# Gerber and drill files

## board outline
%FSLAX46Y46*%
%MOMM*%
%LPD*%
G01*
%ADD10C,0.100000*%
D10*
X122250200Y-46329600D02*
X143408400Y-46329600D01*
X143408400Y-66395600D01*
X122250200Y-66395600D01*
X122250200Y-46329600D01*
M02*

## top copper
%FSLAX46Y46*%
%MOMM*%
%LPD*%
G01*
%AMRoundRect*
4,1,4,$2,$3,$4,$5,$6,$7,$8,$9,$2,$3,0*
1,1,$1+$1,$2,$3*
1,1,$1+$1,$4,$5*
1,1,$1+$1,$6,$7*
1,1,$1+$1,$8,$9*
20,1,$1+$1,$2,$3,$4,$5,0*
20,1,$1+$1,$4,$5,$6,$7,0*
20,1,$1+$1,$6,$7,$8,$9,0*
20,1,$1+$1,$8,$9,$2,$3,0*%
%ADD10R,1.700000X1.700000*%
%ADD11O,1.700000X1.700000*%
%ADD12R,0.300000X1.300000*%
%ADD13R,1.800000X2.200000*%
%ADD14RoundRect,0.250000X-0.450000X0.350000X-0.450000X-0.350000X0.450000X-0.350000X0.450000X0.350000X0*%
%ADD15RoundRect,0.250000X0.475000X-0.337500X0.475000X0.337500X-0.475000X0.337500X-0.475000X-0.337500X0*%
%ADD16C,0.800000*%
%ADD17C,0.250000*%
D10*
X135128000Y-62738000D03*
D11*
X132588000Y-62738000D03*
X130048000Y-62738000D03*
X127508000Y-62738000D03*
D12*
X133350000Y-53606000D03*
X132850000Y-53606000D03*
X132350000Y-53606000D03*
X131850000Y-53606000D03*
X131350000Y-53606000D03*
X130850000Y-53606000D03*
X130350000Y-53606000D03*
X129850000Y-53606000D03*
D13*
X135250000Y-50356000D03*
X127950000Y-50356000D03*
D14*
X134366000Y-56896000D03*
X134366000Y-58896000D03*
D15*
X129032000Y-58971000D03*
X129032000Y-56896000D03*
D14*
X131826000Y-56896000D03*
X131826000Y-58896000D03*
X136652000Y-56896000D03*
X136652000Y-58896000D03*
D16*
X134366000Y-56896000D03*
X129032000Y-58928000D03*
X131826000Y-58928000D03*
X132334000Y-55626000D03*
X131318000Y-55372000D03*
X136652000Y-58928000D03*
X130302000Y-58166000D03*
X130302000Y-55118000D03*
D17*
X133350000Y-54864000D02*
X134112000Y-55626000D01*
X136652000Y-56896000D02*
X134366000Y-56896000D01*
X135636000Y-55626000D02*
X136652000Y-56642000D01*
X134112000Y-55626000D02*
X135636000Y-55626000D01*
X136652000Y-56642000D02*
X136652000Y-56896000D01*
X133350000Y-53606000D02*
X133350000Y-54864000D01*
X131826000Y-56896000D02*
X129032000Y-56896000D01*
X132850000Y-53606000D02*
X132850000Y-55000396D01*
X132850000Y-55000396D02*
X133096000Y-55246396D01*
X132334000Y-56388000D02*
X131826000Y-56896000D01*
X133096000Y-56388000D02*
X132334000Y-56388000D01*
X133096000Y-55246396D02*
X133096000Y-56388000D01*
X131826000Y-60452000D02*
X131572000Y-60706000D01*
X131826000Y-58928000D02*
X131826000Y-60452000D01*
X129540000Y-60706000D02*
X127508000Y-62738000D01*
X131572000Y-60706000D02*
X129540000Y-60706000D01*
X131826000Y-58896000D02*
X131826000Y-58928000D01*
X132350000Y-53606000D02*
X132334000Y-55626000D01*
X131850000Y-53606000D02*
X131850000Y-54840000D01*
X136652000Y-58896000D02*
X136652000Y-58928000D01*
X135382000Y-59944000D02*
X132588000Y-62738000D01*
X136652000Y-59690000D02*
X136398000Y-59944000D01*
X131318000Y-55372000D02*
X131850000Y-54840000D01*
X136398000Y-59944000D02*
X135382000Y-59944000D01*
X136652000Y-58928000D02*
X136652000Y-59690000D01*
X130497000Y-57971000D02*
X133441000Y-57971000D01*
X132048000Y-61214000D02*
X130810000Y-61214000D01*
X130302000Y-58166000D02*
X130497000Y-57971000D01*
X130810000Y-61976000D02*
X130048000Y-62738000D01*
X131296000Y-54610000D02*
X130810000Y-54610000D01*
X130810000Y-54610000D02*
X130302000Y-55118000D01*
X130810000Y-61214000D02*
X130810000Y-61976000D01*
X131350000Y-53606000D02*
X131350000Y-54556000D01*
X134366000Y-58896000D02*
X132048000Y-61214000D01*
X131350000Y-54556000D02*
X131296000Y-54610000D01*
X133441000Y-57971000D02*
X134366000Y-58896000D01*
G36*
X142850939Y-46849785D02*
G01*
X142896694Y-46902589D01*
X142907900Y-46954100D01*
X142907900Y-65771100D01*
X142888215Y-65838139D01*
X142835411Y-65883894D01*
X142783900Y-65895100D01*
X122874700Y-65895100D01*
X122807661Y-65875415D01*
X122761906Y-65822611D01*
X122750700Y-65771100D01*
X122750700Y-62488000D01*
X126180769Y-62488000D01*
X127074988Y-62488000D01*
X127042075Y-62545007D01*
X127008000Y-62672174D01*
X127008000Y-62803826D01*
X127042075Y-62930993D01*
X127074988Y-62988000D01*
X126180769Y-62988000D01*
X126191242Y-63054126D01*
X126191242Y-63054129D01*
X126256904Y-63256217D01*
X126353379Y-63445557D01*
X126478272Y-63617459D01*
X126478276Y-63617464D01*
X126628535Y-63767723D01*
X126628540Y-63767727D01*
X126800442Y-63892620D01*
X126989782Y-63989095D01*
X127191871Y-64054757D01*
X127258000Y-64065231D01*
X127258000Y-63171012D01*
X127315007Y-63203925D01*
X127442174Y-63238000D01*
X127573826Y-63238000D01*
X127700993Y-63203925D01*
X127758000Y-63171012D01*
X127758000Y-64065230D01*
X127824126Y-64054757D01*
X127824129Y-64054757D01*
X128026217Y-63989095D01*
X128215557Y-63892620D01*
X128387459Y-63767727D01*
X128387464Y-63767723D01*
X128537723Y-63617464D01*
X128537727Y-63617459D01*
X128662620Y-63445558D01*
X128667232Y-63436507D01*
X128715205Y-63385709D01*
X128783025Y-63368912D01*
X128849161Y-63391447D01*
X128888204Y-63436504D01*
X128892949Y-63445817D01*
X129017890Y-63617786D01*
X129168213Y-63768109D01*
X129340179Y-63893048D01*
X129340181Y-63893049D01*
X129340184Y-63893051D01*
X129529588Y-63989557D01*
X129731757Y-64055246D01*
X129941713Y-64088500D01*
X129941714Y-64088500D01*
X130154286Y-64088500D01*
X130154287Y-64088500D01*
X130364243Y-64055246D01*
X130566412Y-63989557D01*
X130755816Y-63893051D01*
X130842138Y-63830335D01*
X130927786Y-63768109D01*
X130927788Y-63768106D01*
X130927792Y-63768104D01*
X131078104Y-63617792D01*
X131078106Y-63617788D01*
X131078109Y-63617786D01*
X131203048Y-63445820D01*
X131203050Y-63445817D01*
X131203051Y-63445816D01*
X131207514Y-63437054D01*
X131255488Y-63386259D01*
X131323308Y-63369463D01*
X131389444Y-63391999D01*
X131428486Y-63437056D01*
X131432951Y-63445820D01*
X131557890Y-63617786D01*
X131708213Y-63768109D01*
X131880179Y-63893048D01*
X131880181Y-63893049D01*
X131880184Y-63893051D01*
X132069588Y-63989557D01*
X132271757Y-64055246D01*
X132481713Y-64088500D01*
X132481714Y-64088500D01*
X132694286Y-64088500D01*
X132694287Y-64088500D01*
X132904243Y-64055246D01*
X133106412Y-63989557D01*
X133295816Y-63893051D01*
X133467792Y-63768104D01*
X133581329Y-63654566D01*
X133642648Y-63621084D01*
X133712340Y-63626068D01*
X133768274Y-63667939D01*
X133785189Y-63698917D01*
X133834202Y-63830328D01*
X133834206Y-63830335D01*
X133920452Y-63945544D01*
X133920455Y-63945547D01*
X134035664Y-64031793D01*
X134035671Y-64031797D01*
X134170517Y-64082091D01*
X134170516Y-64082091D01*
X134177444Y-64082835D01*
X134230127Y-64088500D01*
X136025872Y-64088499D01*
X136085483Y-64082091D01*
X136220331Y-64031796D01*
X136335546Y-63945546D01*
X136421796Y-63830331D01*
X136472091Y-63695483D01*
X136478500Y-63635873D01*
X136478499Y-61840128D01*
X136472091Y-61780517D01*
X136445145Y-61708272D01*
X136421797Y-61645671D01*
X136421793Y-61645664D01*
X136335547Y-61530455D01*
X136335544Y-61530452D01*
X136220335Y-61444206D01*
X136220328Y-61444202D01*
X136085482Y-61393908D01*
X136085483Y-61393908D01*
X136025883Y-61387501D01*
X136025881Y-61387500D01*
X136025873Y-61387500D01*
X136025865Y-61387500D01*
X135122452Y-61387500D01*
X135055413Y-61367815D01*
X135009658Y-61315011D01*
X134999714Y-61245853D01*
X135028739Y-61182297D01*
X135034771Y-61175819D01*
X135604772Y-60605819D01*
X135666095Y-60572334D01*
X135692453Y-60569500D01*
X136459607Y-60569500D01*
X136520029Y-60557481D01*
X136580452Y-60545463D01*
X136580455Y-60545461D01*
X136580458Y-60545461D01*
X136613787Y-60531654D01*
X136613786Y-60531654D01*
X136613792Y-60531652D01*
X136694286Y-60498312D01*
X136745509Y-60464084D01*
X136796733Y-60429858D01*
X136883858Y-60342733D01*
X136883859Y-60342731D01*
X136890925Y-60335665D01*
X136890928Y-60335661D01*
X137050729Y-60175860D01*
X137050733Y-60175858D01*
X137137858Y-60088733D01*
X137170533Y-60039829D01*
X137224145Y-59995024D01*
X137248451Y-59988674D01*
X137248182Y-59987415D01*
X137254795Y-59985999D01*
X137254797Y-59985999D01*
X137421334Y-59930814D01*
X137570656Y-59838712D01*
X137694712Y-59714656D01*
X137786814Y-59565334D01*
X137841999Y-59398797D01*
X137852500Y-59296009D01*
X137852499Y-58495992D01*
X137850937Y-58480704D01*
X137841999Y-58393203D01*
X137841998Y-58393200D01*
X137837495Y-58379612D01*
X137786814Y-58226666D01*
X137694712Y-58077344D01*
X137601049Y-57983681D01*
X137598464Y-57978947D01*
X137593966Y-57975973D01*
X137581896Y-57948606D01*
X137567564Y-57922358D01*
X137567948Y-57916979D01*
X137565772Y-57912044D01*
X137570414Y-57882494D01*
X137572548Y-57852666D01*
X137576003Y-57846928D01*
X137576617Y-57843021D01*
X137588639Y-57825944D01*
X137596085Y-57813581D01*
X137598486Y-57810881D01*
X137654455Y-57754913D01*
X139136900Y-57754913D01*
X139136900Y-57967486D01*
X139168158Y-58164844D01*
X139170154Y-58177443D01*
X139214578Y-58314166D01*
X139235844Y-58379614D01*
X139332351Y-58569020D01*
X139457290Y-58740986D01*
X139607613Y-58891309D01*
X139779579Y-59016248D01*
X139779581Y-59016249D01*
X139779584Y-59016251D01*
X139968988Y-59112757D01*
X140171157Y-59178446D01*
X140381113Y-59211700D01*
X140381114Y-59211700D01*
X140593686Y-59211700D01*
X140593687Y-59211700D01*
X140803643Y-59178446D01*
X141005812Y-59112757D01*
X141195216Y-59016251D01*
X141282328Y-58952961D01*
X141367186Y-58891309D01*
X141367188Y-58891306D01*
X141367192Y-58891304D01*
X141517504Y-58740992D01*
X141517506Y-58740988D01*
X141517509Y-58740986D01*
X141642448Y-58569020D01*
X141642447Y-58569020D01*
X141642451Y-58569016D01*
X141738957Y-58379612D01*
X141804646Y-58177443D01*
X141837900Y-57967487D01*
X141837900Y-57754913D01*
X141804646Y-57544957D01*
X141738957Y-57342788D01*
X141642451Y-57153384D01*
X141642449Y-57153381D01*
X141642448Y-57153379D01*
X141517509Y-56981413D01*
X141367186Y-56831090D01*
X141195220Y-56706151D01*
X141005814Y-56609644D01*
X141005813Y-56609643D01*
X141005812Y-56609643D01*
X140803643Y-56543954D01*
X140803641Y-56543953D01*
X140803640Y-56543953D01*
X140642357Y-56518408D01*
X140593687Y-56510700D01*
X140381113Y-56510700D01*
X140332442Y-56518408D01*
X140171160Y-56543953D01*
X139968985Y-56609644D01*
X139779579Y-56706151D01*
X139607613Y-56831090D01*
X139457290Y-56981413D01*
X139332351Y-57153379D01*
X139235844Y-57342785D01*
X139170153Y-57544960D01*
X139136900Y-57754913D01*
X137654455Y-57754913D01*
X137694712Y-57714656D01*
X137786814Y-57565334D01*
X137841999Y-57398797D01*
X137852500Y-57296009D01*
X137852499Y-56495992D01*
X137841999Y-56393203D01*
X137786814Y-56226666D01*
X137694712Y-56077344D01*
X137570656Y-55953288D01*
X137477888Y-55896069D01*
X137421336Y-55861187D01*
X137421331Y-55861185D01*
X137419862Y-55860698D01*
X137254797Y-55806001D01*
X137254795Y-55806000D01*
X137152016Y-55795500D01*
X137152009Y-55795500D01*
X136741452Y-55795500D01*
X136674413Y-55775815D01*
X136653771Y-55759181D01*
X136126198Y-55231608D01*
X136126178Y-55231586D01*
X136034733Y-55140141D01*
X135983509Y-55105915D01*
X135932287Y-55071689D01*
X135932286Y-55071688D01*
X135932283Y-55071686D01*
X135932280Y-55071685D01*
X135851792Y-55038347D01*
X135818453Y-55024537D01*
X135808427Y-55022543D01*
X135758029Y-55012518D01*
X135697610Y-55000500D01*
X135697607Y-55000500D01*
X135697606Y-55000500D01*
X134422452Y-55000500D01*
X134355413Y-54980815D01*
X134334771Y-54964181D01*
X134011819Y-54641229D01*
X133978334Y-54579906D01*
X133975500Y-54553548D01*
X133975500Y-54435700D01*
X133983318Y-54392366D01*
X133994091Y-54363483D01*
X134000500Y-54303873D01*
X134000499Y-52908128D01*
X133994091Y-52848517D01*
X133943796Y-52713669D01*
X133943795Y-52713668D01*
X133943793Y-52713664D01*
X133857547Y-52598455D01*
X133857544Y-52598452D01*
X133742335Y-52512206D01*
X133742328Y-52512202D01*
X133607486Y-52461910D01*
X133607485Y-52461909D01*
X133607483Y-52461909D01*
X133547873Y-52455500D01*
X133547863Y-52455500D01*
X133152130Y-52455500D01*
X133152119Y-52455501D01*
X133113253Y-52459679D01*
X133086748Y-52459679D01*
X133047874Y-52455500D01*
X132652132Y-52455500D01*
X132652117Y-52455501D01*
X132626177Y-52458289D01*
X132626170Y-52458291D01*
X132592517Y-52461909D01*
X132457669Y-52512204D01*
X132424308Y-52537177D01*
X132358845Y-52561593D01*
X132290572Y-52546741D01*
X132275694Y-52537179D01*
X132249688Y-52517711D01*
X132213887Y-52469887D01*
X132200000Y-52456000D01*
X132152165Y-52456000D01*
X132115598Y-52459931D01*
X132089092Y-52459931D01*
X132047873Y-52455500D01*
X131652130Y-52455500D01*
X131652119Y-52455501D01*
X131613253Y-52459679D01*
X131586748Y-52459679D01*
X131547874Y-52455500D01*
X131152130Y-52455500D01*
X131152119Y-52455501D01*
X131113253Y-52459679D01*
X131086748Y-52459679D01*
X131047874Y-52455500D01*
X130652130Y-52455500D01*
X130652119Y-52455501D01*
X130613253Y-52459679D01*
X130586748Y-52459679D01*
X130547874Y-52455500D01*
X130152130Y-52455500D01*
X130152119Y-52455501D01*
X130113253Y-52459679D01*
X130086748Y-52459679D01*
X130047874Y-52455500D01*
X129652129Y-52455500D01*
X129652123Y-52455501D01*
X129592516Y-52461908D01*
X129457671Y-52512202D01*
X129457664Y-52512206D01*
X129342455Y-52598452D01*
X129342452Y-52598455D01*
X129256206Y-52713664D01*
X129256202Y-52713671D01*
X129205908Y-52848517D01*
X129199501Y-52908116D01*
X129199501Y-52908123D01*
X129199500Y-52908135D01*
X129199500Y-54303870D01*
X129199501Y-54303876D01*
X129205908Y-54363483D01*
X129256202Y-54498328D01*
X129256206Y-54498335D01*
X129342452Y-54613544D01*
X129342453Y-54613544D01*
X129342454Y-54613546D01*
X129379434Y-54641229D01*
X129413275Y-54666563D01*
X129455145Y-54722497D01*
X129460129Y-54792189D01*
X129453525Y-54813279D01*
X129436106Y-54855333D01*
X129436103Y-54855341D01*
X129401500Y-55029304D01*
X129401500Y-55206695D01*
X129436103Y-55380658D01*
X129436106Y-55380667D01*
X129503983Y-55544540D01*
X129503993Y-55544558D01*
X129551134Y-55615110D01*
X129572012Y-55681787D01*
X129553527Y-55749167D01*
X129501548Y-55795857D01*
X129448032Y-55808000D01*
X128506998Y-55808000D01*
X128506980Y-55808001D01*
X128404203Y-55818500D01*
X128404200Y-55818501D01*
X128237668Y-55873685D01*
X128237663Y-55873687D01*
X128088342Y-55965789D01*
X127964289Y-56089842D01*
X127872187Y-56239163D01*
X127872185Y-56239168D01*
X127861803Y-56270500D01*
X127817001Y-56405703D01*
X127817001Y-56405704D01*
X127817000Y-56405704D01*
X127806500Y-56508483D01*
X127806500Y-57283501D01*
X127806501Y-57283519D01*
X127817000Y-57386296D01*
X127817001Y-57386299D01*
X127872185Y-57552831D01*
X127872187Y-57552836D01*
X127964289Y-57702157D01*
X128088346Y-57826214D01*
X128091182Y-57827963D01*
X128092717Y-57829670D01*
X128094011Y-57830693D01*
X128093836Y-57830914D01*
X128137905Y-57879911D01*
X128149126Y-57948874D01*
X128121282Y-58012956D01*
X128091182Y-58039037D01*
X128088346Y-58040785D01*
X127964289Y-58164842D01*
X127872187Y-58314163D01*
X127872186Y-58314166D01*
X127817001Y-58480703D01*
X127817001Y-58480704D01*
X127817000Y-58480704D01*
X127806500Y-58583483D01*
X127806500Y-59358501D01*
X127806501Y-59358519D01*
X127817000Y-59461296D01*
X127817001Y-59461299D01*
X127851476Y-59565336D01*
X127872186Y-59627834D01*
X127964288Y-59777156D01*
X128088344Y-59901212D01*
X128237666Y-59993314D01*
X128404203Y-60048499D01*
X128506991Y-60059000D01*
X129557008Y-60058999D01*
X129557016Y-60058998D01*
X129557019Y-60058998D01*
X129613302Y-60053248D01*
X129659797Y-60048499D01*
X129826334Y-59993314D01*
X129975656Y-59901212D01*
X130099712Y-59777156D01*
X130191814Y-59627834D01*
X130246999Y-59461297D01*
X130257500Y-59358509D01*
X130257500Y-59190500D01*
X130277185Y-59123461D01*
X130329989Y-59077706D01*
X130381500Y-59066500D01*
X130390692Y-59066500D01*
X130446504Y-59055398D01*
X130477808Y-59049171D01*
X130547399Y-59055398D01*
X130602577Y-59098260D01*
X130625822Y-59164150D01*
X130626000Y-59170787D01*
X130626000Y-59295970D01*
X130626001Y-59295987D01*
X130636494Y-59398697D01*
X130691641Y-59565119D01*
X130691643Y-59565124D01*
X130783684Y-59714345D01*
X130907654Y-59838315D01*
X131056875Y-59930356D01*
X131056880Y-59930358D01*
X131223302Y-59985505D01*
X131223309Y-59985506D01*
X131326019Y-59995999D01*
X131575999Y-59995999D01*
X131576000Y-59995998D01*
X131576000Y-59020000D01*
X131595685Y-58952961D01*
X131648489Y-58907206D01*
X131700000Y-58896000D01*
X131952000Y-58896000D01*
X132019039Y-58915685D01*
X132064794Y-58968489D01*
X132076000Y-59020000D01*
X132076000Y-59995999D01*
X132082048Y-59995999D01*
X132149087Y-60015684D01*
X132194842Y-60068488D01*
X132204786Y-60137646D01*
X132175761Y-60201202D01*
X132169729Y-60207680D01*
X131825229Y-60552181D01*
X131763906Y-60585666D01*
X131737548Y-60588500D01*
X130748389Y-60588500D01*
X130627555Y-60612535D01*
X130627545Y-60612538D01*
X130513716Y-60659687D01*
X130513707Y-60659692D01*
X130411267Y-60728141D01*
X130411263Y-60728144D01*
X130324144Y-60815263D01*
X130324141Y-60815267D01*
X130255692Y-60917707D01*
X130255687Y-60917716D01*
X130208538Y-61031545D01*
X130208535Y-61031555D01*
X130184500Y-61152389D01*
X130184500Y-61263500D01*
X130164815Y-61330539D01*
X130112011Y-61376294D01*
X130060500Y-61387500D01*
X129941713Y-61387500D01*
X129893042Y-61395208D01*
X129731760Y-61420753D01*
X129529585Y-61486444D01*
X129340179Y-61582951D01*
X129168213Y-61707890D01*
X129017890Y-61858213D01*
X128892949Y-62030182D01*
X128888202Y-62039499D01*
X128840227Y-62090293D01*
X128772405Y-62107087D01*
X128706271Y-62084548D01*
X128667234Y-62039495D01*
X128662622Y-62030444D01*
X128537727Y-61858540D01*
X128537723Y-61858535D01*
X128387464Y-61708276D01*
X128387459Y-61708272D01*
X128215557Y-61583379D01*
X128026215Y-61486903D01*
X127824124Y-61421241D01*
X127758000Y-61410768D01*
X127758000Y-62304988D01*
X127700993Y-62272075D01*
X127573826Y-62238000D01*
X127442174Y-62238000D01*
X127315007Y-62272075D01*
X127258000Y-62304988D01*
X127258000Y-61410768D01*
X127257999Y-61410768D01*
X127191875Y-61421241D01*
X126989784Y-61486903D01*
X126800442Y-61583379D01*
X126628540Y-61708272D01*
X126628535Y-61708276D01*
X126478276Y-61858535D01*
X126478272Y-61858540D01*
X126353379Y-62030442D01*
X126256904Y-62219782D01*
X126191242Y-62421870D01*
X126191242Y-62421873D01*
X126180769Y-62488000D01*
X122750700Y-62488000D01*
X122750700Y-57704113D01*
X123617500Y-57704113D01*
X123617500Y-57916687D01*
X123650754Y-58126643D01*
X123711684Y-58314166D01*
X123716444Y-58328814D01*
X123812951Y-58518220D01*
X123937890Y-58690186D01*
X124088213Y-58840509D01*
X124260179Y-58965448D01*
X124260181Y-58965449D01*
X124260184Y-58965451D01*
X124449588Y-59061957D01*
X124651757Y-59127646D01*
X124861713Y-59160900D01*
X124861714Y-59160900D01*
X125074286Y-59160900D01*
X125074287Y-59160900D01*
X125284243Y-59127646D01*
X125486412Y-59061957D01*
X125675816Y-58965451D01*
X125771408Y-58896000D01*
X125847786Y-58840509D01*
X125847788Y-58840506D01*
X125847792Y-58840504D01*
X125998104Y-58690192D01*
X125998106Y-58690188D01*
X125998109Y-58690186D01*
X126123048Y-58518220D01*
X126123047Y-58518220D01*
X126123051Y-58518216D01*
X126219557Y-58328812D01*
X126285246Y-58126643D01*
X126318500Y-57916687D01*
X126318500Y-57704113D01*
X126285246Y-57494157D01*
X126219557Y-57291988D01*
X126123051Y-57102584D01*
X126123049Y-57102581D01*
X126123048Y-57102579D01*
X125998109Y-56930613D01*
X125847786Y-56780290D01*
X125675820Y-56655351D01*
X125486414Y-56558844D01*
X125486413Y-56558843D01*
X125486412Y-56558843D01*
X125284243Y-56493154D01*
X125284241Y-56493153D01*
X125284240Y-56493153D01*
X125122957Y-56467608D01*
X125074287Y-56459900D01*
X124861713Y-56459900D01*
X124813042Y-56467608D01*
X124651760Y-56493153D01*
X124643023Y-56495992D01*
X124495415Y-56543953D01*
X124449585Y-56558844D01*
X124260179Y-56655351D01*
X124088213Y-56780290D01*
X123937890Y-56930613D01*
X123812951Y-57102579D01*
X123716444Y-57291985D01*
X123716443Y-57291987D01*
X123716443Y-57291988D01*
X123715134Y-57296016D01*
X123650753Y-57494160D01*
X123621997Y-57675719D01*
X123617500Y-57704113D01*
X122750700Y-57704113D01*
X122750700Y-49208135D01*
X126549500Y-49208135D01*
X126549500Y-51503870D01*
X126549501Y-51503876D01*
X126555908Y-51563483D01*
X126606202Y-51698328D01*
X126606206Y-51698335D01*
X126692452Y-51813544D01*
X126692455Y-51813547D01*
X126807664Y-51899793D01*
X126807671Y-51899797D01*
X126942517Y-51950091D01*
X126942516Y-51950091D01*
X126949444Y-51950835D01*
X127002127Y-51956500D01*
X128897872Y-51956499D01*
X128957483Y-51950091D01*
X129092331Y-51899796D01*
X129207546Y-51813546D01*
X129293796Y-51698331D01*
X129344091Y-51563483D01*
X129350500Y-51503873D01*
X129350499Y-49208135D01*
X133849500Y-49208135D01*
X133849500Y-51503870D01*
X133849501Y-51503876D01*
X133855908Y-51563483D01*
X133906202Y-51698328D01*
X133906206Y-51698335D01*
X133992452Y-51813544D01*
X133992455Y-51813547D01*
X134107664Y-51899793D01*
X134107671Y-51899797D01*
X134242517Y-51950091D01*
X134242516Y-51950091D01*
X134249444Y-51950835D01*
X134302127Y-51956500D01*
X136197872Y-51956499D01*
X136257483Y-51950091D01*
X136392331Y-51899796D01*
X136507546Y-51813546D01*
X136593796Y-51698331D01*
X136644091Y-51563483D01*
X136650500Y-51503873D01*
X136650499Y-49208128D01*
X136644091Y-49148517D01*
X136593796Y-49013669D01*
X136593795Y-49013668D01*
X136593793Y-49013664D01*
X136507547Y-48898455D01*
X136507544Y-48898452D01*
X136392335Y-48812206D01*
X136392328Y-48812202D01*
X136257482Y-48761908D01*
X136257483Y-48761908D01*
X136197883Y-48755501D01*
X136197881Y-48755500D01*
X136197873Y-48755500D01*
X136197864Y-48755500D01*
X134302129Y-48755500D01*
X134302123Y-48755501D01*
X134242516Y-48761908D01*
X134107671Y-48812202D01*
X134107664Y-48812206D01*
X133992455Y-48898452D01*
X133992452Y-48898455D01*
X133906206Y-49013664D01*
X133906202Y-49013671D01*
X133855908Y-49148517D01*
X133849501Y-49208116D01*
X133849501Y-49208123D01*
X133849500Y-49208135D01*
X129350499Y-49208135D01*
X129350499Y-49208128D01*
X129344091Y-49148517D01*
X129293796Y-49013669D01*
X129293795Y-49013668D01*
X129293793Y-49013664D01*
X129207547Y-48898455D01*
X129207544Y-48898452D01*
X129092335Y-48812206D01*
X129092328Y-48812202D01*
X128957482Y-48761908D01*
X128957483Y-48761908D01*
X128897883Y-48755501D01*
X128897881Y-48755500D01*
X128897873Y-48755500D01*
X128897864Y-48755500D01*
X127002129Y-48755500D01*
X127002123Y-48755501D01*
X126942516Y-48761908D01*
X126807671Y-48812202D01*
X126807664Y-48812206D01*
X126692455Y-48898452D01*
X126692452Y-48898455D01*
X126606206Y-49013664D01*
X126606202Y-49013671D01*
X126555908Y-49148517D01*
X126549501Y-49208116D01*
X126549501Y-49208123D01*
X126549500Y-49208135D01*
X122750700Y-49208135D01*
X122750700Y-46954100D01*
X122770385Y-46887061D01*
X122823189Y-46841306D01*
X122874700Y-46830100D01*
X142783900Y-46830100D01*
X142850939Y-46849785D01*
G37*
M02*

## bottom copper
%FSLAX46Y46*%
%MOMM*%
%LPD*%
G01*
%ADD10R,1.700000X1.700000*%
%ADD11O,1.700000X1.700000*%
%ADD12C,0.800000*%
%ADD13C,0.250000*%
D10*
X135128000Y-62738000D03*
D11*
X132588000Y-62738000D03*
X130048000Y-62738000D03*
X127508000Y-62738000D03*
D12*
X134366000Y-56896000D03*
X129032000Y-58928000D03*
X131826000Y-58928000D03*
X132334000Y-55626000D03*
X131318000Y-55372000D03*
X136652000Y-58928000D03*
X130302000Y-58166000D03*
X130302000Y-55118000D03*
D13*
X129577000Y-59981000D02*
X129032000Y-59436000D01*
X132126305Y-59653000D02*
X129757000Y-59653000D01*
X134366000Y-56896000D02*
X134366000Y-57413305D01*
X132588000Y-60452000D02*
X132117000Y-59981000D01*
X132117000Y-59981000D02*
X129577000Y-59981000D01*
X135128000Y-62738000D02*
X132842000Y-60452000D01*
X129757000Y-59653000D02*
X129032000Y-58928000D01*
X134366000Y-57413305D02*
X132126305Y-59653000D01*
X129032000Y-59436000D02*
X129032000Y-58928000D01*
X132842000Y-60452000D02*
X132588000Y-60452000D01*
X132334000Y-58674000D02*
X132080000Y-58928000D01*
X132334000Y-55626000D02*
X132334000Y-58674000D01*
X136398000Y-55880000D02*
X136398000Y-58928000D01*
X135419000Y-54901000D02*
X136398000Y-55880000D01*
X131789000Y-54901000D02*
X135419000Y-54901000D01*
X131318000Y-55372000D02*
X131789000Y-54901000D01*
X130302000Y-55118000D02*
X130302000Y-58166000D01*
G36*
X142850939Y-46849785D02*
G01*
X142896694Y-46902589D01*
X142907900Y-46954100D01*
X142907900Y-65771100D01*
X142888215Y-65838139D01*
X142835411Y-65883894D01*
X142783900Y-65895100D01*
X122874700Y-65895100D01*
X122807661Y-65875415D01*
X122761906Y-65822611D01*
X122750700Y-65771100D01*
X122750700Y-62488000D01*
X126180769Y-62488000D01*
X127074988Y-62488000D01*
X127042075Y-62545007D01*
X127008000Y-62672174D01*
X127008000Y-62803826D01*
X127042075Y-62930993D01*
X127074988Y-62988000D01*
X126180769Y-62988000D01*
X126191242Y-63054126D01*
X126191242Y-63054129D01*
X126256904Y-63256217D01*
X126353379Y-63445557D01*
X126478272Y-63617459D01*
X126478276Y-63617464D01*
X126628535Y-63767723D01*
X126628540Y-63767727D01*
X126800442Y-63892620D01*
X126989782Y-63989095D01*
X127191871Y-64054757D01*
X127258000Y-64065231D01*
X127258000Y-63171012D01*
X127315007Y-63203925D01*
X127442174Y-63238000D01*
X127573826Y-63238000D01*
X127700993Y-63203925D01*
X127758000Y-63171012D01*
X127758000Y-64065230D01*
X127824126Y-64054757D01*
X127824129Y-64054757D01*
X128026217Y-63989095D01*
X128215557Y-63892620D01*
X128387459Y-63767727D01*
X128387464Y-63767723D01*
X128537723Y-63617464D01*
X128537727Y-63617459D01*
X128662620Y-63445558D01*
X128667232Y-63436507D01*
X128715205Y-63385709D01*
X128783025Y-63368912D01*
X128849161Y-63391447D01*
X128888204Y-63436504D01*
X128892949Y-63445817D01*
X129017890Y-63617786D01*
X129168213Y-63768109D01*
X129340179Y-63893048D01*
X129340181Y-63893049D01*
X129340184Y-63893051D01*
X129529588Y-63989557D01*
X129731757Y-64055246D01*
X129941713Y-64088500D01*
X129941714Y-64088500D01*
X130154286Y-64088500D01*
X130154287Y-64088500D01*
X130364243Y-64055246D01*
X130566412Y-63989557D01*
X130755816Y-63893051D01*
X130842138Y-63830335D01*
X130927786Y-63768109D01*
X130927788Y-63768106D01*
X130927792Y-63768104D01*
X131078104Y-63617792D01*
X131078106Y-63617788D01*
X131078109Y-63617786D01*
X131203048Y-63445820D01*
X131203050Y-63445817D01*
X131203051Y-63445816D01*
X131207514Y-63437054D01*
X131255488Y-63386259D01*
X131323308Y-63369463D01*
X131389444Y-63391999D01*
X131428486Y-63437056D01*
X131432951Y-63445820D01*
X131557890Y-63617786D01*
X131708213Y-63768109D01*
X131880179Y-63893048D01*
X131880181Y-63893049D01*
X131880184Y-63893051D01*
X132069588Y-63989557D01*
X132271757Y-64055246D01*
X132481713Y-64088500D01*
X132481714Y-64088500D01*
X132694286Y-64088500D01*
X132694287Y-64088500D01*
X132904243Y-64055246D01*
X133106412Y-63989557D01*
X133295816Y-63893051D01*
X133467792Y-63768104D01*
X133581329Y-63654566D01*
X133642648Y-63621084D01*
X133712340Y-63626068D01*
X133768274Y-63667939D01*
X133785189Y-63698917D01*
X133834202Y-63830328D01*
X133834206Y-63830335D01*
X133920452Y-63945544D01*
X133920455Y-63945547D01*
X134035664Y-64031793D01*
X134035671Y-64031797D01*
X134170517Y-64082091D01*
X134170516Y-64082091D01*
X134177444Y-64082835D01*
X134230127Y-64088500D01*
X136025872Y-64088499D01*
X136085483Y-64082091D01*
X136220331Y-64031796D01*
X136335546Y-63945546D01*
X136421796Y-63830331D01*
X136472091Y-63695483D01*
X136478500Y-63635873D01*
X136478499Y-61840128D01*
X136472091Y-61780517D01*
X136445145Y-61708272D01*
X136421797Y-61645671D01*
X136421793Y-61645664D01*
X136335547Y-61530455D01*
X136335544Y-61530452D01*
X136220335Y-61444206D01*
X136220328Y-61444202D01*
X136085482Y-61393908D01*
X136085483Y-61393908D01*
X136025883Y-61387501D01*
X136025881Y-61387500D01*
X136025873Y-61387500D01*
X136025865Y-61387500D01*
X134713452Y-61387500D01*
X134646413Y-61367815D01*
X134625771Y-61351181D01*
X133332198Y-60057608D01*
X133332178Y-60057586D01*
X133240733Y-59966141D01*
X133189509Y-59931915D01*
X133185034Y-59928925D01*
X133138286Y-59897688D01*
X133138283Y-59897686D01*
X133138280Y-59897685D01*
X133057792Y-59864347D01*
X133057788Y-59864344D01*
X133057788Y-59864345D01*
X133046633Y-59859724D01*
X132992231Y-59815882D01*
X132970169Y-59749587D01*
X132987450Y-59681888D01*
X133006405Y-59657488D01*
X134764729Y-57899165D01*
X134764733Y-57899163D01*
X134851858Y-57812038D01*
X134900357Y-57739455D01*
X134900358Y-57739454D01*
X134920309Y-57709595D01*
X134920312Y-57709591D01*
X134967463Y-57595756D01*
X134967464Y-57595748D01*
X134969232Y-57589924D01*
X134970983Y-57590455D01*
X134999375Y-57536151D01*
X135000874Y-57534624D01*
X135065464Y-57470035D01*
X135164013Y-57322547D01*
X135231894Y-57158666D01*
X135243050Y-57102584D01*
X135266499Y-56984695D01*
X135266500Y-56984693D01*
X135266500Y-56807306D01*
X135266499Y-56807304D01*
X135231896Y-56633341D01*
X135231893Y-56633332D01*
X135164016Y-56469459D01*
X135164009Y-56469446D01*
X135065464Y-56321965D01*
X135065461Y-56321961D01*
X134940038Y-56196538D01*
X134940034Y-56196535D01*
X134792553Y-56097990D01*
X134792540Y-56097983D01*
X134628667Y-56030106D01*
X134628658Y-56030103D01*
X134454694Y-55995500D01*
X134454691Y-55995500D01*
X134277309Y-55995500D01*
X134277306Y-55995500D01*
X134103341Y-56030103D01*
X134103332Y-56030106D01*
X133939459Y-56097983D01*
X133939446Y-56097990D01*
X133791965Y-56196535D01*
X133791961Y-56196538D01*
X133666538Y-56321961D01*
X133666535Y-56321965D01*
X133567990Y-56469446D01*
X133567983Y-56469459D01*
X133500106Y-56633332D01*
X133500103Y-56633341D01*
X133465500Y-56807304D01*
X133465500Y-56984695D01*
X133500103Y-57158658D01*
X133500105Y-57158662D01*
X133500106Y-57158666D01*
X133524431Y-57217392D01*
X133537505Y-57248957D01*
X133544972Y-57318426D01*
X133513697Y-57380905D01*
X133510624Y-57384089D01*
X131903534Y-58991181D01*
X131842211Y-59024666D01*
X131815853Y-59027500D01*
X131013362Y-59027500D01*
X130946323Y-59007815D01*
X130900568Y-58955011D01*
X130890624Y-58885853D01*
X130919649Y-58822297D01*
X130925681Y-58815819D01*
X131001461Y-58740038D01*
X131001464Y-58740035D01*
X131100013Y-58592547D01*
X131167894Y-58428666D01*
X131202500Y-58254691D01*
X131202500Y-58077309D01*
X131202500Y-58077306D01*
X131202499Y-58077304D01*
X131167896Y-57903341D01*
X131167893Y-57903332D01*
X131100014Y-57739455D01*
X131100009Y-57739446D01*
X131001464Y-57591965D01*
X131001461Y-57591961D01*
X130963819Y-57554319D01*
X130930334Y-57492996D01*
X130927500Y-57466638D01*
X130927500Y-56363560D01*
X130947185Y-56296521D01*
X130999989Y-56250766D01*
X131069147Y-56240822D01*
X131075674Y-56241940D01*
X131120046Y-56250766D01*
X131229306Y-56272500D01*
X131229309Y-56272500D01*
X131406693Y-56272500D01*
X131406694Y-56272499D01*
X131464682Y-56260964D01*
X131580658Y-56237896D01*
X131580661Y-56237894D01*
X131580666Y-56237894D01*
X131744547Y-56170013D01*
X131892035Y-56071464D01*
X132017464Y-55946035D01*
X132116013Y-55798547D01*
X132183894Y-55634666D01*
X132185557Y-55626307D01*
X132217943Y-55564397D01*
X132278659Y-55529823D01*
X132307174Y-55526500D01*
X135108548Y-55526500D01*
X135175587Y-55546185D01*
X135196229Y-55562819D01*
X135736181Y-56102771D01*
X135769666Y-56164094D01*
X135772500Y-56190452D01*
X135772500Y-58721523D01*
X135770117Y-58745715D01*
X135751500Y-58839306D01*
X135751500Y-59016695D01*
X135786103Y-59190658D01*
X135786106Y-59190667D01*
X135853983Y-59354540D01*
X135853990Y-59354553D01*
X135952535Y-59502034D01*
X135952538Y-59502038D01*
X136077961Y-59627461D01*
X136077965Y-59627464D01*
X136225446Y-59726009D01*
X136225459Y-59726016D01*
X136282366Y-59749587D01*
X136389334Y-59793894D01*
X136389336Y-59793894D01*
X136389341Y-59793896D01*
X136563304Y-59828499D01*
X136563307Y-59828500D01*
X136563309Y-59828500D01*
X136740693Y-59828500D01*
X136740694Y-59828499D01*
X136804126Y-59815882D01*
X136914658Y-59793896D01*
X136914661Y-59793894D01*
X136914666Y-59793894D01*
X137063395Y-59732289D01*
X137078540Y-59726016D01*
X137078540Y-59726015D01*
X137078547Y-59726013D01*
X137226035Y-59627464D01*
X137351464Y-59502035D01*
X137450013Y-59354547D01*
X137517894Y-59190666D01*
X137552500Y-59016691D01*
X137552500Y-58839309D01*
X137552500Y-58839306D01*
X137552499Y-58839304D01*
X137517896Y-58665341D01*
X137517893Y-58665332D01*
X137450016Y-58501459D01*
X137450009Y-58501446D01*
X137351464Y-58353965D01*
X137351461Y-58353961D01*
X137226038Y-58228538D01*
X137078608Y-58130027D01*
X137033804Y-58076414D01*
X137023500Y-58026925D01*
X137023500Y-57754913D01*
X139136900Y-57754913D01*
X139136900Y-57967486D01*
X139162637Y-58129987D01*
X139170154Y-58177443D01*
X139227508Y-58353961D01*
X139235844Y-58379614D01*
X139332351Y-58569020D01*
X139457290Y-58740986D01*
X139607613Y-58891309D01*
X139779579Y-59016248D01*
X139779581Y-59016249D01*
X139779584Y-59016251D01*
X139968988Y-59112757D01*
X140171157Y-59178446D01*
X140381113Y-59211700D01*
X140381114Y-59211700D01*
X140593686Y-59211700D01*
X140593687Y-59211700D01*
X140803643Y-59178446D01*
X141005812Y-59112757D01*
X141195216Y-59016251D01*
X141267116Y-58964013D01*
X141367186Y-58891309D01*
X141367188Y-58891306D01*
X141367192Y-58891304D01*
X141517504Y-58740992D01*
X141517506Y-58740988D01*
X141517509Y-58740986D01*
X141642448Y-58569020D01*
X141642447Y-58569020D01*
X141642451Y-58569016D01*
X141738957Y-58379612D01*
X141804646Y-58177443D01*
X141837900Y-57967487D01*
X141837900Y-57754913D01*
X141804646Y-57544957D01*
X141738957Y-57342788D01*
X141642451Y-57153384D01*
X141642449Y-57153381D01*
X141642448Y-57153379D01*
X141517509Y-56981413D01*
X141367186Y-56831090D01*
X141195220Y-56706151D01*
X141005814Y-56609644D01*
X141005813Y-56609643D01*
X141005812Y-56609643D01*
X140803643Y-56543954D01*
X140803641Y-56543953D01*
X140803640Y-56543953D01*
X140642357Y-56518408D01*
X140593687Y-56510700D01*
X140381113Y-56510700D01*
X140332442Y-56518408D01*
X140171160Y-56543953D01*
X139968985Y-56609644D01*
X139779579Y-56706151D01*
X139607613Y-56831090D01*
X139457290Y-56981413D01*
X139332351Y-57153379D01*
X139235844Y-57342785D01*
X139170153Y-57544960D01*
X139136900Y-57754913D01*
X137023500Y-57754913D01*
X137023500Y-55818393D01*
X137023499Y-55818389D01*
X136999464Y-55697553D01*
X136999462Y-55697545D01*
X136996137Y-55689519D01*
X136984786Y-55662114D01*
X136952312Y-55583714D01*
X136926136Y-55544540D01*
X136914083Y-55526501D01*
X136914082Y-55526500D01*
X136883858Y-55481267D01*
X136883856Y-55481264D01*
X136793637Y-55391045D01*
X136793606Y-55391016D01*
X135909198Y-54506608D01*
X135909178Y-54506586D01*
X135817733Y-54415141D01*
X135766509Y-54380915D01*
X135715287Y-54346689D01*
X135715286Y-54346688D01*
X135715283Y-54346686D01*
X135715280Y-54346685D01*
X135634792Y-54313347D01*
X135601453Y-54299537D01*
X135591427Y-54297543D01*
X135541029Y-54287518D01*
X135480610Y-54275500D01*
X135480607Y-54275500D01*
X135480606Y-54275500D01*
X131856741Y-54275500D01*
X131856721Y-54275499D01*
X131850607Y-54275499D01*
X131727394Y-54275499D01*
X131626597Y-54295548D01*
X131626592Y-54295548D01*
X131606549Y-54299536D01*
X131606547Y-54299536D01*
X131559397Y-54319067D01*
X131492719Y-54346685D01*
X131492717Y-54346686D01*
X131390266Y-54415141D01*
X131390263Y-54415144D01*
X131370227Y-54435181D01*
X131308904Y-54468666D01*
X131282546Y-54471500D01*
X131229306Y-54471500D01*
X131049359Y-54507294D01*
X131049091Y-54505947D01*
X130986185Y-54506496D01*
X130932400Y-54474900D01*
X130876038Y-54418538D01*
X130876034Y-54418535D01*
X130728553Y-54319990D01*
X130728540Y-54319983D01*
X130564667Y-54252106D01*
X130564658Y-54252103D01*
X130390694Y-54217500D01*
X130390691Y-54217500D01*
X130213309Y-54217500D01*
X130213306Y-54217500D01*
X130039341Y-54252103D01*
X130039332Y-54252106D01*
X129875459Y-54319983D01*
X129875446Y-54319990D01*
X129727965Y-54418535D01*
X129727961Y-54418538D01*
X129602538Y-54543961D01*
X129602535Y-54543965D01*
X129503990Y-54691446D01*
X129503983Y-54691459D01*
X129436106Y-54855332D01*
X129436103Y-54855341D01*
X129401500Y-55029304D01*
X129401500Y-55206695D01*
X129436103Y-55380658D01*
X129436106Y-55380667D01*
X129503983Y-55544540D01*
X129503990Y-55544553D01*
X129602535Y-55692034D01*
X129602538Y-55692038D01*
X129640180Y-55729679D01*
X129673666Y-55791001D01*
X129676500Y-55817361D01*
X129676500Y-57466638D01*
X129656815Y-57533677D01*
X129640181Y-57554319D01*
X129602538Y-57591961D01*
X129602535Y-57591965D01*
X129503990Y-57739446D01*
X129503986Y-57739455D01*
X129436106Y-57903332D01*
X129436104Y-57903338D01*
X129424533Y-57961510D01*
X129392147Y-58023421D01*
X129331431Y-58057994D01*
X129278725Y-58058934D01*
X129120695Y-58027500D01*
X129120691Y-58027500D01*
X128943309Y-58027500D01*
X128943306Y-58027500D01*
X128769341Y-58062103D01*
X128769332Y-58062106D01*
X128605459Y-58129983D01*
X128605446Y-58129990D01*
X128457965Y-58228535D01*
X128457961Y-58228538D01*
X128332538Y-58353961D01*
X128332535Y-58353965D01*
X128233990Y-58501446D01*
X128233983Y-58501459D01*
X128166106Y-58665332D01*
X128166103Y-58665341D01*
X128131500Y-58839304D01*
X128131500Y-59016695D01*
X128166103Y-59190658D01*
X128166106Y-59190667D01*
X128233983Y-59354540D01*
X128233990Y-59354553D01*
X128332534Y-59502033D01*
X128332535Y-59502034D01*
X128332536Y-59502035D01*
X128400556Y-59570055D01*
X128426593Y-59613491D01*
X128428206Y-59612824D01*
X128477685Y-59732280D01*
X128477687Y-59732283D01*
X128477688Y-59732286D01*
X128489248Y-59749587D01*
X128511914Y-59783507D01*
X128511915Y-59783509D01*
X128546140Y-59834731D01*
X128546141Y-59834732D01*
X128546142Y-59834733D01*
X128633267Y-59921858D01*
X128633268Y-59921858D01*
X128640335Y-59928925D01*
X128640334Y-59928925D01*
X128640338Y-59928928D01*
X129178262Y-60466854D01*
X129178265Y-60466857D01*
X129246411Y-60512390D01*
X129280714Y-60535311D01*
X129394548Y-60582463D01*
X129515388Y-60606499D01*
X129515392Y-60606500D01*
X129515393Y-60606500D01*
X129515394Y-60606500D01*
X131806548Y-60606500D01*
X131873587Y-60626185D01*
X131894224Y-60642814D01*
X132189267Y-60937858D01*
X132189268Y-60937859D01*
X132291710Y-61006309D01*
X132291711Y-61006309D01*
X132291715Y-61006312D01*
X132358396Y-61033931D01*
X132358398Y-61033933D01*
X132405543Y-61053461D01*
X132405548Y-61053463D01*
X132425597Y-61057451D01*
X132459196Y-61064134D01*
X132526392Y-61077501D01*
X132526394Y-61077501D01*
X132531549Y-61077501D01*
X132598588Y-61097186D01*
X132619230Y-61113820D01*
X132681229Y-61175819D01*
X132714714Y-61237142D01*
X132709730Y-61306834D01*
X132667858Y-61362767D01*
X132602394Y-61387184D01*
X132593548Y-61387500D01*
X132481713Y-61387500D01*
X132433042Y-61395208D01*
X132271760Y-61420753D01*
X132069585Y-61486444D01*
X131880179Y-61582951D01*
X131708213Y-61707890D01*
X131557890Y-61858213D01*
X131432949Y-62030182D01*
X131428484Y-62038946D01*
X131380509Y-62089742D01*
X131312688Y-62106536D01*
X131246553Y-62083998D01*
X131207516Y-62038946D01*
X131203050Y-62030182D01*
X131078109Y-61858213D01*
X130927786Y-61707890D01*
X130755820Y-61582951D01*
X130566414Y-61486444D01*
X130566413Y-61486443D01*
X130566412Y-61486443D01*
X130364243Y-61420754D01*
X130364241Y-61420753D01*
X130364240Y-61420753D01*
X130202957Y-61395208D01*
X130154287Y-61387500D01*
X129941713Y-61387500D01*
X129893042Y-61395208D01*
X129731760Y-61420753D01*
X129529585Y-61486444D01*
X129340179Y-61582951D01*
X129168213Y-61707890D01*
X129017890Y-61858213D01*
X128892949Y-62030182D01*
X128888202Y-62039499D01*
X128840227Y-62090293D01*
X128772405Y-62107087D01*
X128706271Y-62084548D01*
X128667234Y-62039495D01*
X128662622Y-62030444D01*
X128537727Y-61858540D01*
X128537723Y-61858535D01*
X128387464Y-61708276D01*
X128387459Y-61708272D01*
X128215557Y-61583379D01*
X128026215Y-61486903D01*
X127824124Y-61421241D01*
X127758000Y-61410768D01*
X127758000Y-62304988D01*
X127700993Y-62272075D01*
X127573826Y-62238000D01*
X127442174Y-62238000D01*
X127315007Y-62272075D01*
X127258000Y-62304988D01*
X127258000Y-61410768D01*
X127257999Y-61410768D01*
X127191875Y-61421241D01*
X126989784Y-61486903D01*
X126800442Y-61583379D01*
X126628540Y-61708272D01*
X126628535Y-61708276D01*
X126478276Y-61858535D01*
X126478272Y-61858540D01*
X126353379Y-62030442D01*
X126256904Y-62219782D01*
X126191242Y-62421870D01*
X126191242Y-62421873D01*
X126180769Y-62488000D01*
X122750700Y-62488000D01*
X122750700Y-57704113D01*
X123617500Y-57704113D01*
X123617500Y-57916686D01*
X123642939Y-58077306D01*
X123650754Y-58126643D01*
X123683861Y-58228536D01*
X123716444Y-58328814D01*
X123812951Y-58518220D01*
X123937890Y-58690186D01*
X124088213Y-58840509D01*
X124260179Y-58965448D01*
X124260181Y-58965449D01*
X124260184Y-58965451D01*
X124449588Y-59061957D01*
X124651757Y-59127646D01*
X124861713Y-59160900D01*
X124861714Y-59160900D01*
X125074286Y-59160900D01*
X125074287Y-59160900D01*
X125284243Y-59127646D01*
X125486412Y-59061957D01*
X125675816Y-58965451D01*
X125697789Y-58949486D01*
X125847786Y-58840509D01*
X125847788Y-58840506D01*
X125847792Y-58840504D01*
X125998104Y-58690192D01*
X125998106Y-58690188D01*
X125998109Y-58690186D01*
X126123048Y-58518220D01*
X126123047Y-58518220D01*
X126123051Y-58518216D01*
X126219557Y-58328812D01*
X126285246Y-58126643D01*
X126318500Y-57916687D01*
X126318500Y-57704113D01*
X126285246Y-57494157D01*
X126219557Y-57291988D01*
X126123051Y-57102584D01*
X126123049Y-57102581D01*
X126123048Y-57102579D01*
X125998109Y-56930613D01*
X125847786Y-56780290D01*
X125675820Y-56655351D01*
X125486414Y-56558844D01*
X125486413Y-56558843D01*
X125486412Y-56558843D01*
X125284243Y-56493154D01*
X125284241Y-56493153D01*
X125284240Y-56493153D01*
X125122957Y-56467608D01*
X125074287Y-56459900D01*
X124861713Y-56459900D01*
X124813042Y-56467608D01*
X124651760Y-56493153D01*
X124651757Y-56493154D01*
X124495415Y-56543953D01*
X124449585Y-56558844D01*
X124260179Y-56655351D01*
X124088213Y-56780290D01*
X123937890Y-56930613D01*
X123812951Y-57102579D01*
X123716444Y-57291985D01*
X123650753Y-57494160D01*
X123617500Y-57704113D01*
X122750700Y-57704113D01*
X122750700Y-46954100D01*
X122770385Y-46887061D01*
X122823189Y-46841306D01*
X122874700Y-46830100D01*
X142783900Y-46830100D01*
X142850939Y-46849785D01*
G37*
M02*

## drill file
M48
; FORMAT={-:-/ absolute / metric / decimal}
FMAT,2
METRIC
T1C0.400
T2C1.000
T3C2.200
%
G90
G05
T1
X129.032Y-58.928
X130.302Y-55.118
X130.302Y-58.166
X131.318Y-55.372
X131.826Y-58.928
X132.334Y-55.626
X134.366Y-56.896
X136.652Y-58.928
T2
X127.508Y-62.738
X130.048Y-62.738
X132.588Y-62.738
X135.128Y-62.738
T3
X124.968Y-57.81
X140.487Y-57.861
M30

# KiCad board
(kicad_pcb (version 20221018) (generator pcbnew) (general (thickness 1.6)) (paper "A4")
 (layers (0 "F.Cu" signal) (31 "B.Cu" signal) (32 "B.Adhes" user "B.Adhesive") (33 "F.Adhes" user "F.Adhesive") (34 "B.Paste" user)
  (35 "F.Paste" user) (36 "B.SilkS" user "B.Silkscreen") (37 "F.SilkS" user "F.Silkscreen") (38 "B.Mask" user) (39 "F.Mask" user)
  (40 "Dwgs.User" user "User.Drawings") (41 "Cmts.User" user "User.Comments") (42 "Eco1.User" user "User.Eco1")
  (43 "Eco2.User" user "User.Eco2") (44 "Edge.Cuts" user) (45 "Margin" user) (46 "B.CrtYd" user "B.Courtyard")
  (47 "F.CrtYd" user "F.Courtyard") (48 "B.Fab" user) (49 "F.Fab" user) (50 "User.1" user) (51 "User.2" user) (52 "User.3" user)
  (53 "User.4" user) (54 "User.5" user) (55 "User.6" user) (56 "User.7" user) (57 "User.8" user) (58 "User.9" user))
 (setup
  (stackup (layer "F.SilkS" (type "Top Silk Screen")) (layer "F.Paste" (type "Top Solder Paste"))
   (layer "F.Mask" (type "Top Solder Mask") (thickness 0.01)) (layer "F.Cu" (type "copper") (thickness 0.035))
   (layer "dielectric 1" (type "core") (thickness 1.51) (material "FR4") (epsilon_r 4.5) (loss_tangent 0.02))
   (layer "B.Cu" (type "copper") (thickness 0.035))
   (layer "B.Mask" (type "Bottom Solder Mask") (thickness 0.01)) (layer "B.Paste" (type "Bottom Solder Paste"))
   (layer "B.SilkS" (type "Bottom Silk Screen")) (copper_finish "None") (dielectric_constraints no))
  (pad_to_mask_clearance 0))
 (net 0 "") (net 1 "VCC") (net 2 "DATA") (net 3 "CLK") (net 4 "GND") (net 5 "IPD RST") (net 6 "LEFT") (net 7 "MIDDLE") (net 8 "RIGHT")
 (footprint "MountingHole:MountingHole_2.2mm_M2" (layer "F.Cu") (at 140.4874 57.8612)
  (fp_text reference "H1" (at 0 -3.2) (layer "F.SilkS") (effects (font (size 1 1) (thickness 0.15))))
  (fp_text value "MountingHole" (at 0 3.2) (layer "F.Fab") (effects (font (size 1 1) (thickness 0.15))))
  (pad "" np_thru_hole circle (at 0 0) (size 2.2 2.2) (drill 2.2) (layers "*.Cu" "*.Mask")))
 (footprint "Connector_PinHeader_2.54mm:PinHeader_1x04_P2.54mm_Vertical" (layer "F.Cu") (at 135.128 62.738 -90)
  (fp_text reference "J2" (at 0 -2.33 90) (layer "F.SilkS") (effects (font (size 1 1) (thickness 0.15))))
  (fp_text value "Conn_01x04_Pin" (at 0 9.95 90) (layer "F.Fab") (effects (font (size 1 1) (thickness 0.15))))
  (pad "1" thru_hole rect (at 0 0 270) (size 1.7 1.7) (drill 1) (layers "*.Cu" "*.Mask") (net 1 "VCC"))
  (pad "2" thru_hole oval (at 0 2.54 270) (size 1.7 1.7) (drill 1) (layers "*.Cu" "*.Mask") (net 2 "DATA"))
  (pad "3" thru_hole oval (at 0 5.08 270) (size 1.7 1.7) (drill 1) (layers "*.Cu" "*.Mask") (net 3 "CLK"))
  (pad "4" thru_hole oval (at 0 7.62 270) (size 1.7 1.7) (drill 1) (layers "*.Cu" "*.Mask") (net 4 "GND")))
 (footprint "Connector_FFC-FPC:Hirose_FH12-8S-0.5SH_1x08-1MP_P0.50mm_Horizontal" (layer "F.Cu") (at 131.6 51.756 180)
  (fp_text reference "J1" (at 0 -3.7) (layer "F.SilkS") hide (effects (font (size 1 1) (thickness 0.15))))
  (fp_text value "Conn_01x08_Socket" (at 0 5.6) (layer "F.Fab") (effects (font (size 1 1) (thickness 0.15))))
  (pad "1" smd rect (at -1.75 -1.85 180) (size 0.3 1.3) (layers "F.Cu" "F.Paste" "F.Mask") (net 1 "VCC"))
  (pad "2" smd rect (at -1.25 -1.85 180) (size 0.3 1.3) (layers "F.Cu" "F.Paste" "F.Mask") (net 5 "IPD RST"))
  (pad "3" smd rect (at -0.75 -1.85 180) (size 0.3 1.3) (layers "F.Cu" "F.Paste" "F.Mask") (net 4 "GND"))
  (pad "4" smd rect (at -0.25 -1.85 180) (size 0.3 1.3) (layers "F.Cu" "F.Paste" "F.Mask") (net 2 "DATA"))
  (pad "5" smd rect (at 0.25 -1.85 180) (size 0.3 1.3) (layers "F.Cu" "F.Paste" "F.Mask") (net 3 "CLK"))
  (pad "6" smd rect (at 0.75 -1.85 180) (size 0.3 1.3) (layers "F.Cu" "F.Paste" "F.Mask") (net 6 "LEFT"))
  (pad "7" smd rect (at 1.25 -1.85 180) (size 0.3 1.3) (layers "F.Cu" "F.Paste" "F.Mask") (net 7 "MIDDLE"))
  (pad "8" smd rect (at 1.75 -1.85 180) (size 0.3 1.3) (layers "F.Cu" "F.Paste" "F.Mask") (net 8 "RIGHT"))
  (pad "MP" smd rect (at -3.65 1.4 180) (size 1.8 2.2) (layers "F.Cu" "F.Paste" "F.Mask"))
  (pad "MP" smd rect (at 3.65 1.4 180) (size 1.8 2.2) (layers "F.Cu" "F.Paste" "F.Mask")))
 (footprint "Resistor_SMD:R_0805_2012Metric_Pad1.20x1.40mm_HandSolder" (layer "F.Cu") (at 134.366 57.896 -90)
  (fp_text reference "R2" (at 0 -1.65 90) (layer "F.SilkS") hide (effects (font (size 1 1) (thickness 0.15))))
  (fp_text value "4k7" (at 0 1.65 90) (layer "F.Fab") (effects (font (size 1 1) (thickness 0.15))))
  (pad "1" smd roundrect (at -1 0 270) (size 1.2 1.4) (layers "F.Cu" "F.Paste" "F.Mask") (roundrect_rratio 0.2083333333) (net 1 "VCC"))
  (pad "2" smd roundrect (at 1 0 270) (size 1.2 1.4) (layers "F.Cu" "F.Paste" "F.Mask") (roundrect_rratio 0.2083333333) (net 3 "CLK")))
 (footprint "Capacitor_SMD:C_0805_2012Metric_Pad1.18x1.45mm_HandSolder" (layer "F.Cu") (at 129.032 57.9335 90)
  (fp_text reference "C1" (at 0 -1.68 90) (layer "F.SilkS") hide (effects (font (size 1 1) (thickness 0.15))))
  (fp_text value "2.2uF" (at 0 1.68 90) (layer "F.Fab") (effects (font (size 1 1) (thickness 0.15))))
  (pad "1" smd roundrect (at -1.0375 0 90) (size 1.175 1.45) (layers "F.Cu" "F.Paste" "F.Mask") (roundrect_rratio 0.2127659574)
   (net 1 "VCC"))
  (pad "2" smd roundrect (at 1.0375 0 90) (size 1.175 1.45) (layers "F.Cu" "F.Paste" "F.Mask") (roundrect_rratio 0.2127659574)
   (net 5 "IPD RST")))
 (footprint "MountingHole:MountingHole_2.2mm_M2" (layer "F.Cu") (at 124.968 57.8104)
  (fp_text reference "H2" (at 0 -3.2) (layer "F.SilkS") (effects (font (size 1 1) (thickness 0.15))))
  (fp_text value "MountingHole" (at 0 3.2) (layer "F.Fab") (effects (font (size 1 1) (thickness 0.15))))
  (pad "" np_thru_hole circle (at 0 0) (size 2.2 2.2) (drill 2.2) (layers "*.Cu" "*.Mask")))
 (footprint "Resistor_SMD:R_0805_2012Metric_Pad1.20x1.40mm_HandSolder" (layer "F.Cu") (at 131.826 57.896 -90)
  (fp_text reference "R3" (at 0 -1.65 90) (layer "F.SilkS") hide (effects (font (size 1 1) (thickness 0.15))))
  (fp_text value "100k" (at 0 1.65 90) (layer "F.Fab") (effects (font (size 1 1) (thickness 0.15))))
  (pad "1" smd roundrect (at -1 0 270) (size 1.2 1.4) (layers "F.Cu" "F.Paste" "F.Mask") (roundrect_rratio 0.2083333333) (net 5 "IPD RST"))
  (pad "2" smd roundrect (at 1 0 270) (size 1.2 1.4) (layers "F.Cu" "F.Paste" "F.Mask") (roundrect_rratio 0.2083333333) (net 4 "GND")))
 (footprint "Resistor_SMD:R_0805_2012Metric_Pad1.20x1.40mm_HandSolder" (layer "F.Cu") (at 136.652 57.896 -90)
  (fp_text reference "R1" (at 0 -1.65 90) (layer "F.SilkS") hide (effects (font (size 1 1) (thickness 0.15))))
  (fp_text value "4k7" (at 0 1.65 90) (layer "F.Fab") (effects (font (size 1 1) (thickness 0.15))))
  (pad "1" smd roundrect (at -1 0 270) (size 1.2 1.4) (layers "F.Cu" "F.Paste" "F.Mask") (roundrect_rratio 0.2083333333) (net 1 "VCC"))
  (pad "2" smd roundrect (at 1 0 270) (size 1.2 1.4) (layers "F.Cu" "F.Paste" "F.Mask") (roundrect_rratio 0.2083333333) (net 2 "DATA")))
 (gr_rect (start 122.2502 46.3296) (end 143.4084 66.3956) (stroke (width 0.1) (type default)) (fill none) (layer "Edge.Cuts"))
 (segment (start 133.35 54.864) (end 134.112 55.626) (width 0.25) (layer "F.Cu") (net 1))
 (segment (start 136.652 56.896) (end 134.366 56.896) (width 0.25) (layer "F.Cu") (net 1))
 (segment (start 135.636 55.626) (end 136.652 56.642) (width 0.25) (layer "F.Cu") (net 1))
 (segment (start 134.112 55.626) (end 135.636 55.626) (width 0.25) (layer "F.Cu") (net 1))
 (segment (start 136.652 56.642) (end 136.652 56.896) (width 0.25) (layer "F.Cu") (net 1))
 (segment (start 133.35 53.606) (end 133.35 54.864) (width 0.25) (layer "F.Cu") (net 1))
 (via (at 134.366 56.896) (size 0.8) (drill 0.4) (layers "F.Cu" "B.Cu") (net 1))
 (via (at 129.032 58.928) (size 0.8) (drill 0.4) (layers "F.Cu" "B.Cu") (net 1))
 (segment (start 129.577 59.981) (end 129.032 59.436) (width 0.25) (layer "B.Cu") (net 1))
 (segment (start 132.126305 59.653) (end 129.757 59.653) (width 0.25) (layer "B.Cu") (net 1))
 (segment (start 134.366 56.896) (end 134.366 57.413305) (width 0.25) (layer "B.Cu") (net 1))
 (segment (start 132.588 60.452) (end 132.117 59.981) (width 0.25) (layer "B.Cu") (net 1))
 (segment (start 132.117 59.981) (end 129.577 59.981) (width 0.25) (layer "B.Cu") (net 1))
 (segment (start 135.128 62.738) (end 132.842 60.452) (width 0.25) (layer "B.Cu") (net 1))
 (segment (start 129.757 59.653) (end 129.032 58.928) (width 0.25) (layer "B.Cu") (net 1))
 (segment (start 134.366 57.413305) (end 132.126305 59.653) (width 0.25) (layer "B.Cu") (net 1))
 (segment (start 129.032 59.436) (end 129.032 58.928) (width 0.25) (layer "B.Cu") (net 1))
 (segment (start 132.842 60.452) (end 132.588 60.452) (width 0.25) (layer "B.Cu") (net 1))
 (segment (start 131.826 56.896) (end 129.032 56.896) (width 0.25) (layer "F.Cu") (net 5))
 (segment (start 132.85 53.606) (end 132.85 55.000396) (width 0.25) (layer "F.Cu") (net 5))
 (segment (start 132.85 55.000396) (end 133.096 55.246396) (width 0.25) (layer "F.Cu") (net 5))
 (segment (start 132.334 56.388) (end 131.826 56.896) (width 0.25) (layer "F.Cu") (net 5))
 (segment (start 133.096 56.388) (end 132.334 56.388) (width 0.25) (layer "F.Cu") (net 5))
 (segment (start 133.096 55.246396) (end 133.096 56.388) (width 0.25) (layer "F.Cu") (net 5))
 (segment (start 131.826 60.452) (end 131.572 60.706) (width 0.25) (layer "F.Cu") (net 4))
 (segment (start 131.826 58.928) (end 131.826 60.452) (width 0.25) (layer "F.Cu") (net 4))
 (segment (start 129.54 60.706) (end 127.508 62.738) (width 0.25) (layer "F.Cu") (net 4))
 (segment (start 131.572 60.706) (end 129.54 60.706) (width 0.25) (layer "F.Cu") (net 4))
 (segment (start 131.826 58.896) (end 131.826 58.928) (width 0.25) (layer "F.Cu") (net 4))
 (segment (start 132.35 53.606) (end 132.334 55.626) (width 0.25) (layer "F.Cu") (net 4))
 (via (at 131.826 58.928) (size 0.8) (drill 0.4) (layers "F.Cu" "B.Cu") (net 4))
 (via (at 132.334 55.626) (size 0.8) (drill 0.4) (layers "F.Cu" "B.Cu") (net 4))
 (segment (start 132.334 58.674) (end 132.08 58.928) (width 0.25) (layer "B.Cu") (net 4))
 (segment (start 132.334 55.626) (end 132.334 58.674) (width 0.25) (layer "B.Cu") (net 4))
 (segment (start 131.85 53.606) (end 131.85 54.84) (width 0.25) (layer "F.Cu") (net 2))
 (segment (start 136.652 58.896) (end 136.652 58.928) (width 0.25) (layer "F.Cu") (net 2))
 (segment (start 135.382 59.944) (end 132.588 62.738) (width 0.25) (layer "F.Cu") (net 2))
 (segment (start 136.652 59.69) (end 136.398 59.944) (width 0.25) (layer "F.Cu") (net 2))
 (segment (start 131.318 55.372) (end 131.85 54.84) (width 0.25) (layer "F.Cu") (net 2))
 (segment (start 136.398 59.944) (end 135.382 59.944) (width 0.25) (layer "F.Cu") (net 2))
 (segment (start 136.652 58.928) (end 136.652 59.69) (width 0.25) (layer "F.Cu") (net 2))
 (via (at 131.318 55.372) (size 0.8) (drill 0.4) (layers "F.Cu" "B.Cu") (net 2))
 (via (at 136.652 58.928) (size 0.8) (drill 0.4) (layers "F.Cu" "B.Cu") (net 2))
 (segment (start 136.398 55.88) (end 136.398 58.928) (width 0.25) (layer "B.Cu") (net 2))
 (segment (start 135.419 54.901) (end 136.398 55.88) (width 0.25) (layer "B.Cu") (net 2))
 (segment (start 131.789 54.901) (end 135.419 54.901) (width 0.25) (layer "B.Cu") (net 2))
 (segment (start 131.318 55.372) (end 131.789 54.901) (width 0.25) (layer "B.Cu") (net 2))
 (segment (start 130.497 57.971) (end 133.441 57.971) (width 0.25) (layer "F.Cu") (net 3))
 (segment (start 132.048 61.214) (end 130.81 61.214) (width 0.25) (layer "F.Cu") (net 3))
 (segment (start 130.302 58.166) (end 130.497 57.971) (width 0.25) (layer "F.Cu") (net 3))
 (segment (start 130.81 61.976) (end 130.048 62.738) (width 0.25) (layer "F.Cu") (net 3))
 (segment (start 131.296 54.61) (end 130.81 54.61) (width 0.25) (layer "F.Cu") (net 3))
 (segment (start 130.81 54.61) (end 130.302 55.118) (width 0.25) (layer "F.Cu") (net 3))
 (segment (start 130.81 61.214) (end 130.81 61.976) (width 0.25) (layer "F.Cu") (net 3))
 (segment (start 131.35 53.606) (end 131.35 54.556) (width 0.25) (layer "F.Cu") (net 3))
 (segment (start 134.366 58.896) (end 132.048 61.214) (width 0.25) (layer "F.Cu") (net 3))
 (segment (start 131.35 54.556) (end 131.296 54.61) (width 0.25) (layer "F.Cu") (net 3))
 (segment (start 133.441 57.971) (end 134.366 58.896) (width 0.25) (layer "F.Cu") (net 3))
 (via (at 130.302 58.166) (size 0.8) (drill 0.4) (layers "F.Cu" "B.Cu") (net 3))
 (via (at 130.302 55.118) (size 0.8) (drill 0.4) (layers "F.Cu" "B.Cu") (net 3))
 (segment (start 130.302 55.118) (end 130.302 58.166) (width 0.25) (layer "B.Cu") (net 3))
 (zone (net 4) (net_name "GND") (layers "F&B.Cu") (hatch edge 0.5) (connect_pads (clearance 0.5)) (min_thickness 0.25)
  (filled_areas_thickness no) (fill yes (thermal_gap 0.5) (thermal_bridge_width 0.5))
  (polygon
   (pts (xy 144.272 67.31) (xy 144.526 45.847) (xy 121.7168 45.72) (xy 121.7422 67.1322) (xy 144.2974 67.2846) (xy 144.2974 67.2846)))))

